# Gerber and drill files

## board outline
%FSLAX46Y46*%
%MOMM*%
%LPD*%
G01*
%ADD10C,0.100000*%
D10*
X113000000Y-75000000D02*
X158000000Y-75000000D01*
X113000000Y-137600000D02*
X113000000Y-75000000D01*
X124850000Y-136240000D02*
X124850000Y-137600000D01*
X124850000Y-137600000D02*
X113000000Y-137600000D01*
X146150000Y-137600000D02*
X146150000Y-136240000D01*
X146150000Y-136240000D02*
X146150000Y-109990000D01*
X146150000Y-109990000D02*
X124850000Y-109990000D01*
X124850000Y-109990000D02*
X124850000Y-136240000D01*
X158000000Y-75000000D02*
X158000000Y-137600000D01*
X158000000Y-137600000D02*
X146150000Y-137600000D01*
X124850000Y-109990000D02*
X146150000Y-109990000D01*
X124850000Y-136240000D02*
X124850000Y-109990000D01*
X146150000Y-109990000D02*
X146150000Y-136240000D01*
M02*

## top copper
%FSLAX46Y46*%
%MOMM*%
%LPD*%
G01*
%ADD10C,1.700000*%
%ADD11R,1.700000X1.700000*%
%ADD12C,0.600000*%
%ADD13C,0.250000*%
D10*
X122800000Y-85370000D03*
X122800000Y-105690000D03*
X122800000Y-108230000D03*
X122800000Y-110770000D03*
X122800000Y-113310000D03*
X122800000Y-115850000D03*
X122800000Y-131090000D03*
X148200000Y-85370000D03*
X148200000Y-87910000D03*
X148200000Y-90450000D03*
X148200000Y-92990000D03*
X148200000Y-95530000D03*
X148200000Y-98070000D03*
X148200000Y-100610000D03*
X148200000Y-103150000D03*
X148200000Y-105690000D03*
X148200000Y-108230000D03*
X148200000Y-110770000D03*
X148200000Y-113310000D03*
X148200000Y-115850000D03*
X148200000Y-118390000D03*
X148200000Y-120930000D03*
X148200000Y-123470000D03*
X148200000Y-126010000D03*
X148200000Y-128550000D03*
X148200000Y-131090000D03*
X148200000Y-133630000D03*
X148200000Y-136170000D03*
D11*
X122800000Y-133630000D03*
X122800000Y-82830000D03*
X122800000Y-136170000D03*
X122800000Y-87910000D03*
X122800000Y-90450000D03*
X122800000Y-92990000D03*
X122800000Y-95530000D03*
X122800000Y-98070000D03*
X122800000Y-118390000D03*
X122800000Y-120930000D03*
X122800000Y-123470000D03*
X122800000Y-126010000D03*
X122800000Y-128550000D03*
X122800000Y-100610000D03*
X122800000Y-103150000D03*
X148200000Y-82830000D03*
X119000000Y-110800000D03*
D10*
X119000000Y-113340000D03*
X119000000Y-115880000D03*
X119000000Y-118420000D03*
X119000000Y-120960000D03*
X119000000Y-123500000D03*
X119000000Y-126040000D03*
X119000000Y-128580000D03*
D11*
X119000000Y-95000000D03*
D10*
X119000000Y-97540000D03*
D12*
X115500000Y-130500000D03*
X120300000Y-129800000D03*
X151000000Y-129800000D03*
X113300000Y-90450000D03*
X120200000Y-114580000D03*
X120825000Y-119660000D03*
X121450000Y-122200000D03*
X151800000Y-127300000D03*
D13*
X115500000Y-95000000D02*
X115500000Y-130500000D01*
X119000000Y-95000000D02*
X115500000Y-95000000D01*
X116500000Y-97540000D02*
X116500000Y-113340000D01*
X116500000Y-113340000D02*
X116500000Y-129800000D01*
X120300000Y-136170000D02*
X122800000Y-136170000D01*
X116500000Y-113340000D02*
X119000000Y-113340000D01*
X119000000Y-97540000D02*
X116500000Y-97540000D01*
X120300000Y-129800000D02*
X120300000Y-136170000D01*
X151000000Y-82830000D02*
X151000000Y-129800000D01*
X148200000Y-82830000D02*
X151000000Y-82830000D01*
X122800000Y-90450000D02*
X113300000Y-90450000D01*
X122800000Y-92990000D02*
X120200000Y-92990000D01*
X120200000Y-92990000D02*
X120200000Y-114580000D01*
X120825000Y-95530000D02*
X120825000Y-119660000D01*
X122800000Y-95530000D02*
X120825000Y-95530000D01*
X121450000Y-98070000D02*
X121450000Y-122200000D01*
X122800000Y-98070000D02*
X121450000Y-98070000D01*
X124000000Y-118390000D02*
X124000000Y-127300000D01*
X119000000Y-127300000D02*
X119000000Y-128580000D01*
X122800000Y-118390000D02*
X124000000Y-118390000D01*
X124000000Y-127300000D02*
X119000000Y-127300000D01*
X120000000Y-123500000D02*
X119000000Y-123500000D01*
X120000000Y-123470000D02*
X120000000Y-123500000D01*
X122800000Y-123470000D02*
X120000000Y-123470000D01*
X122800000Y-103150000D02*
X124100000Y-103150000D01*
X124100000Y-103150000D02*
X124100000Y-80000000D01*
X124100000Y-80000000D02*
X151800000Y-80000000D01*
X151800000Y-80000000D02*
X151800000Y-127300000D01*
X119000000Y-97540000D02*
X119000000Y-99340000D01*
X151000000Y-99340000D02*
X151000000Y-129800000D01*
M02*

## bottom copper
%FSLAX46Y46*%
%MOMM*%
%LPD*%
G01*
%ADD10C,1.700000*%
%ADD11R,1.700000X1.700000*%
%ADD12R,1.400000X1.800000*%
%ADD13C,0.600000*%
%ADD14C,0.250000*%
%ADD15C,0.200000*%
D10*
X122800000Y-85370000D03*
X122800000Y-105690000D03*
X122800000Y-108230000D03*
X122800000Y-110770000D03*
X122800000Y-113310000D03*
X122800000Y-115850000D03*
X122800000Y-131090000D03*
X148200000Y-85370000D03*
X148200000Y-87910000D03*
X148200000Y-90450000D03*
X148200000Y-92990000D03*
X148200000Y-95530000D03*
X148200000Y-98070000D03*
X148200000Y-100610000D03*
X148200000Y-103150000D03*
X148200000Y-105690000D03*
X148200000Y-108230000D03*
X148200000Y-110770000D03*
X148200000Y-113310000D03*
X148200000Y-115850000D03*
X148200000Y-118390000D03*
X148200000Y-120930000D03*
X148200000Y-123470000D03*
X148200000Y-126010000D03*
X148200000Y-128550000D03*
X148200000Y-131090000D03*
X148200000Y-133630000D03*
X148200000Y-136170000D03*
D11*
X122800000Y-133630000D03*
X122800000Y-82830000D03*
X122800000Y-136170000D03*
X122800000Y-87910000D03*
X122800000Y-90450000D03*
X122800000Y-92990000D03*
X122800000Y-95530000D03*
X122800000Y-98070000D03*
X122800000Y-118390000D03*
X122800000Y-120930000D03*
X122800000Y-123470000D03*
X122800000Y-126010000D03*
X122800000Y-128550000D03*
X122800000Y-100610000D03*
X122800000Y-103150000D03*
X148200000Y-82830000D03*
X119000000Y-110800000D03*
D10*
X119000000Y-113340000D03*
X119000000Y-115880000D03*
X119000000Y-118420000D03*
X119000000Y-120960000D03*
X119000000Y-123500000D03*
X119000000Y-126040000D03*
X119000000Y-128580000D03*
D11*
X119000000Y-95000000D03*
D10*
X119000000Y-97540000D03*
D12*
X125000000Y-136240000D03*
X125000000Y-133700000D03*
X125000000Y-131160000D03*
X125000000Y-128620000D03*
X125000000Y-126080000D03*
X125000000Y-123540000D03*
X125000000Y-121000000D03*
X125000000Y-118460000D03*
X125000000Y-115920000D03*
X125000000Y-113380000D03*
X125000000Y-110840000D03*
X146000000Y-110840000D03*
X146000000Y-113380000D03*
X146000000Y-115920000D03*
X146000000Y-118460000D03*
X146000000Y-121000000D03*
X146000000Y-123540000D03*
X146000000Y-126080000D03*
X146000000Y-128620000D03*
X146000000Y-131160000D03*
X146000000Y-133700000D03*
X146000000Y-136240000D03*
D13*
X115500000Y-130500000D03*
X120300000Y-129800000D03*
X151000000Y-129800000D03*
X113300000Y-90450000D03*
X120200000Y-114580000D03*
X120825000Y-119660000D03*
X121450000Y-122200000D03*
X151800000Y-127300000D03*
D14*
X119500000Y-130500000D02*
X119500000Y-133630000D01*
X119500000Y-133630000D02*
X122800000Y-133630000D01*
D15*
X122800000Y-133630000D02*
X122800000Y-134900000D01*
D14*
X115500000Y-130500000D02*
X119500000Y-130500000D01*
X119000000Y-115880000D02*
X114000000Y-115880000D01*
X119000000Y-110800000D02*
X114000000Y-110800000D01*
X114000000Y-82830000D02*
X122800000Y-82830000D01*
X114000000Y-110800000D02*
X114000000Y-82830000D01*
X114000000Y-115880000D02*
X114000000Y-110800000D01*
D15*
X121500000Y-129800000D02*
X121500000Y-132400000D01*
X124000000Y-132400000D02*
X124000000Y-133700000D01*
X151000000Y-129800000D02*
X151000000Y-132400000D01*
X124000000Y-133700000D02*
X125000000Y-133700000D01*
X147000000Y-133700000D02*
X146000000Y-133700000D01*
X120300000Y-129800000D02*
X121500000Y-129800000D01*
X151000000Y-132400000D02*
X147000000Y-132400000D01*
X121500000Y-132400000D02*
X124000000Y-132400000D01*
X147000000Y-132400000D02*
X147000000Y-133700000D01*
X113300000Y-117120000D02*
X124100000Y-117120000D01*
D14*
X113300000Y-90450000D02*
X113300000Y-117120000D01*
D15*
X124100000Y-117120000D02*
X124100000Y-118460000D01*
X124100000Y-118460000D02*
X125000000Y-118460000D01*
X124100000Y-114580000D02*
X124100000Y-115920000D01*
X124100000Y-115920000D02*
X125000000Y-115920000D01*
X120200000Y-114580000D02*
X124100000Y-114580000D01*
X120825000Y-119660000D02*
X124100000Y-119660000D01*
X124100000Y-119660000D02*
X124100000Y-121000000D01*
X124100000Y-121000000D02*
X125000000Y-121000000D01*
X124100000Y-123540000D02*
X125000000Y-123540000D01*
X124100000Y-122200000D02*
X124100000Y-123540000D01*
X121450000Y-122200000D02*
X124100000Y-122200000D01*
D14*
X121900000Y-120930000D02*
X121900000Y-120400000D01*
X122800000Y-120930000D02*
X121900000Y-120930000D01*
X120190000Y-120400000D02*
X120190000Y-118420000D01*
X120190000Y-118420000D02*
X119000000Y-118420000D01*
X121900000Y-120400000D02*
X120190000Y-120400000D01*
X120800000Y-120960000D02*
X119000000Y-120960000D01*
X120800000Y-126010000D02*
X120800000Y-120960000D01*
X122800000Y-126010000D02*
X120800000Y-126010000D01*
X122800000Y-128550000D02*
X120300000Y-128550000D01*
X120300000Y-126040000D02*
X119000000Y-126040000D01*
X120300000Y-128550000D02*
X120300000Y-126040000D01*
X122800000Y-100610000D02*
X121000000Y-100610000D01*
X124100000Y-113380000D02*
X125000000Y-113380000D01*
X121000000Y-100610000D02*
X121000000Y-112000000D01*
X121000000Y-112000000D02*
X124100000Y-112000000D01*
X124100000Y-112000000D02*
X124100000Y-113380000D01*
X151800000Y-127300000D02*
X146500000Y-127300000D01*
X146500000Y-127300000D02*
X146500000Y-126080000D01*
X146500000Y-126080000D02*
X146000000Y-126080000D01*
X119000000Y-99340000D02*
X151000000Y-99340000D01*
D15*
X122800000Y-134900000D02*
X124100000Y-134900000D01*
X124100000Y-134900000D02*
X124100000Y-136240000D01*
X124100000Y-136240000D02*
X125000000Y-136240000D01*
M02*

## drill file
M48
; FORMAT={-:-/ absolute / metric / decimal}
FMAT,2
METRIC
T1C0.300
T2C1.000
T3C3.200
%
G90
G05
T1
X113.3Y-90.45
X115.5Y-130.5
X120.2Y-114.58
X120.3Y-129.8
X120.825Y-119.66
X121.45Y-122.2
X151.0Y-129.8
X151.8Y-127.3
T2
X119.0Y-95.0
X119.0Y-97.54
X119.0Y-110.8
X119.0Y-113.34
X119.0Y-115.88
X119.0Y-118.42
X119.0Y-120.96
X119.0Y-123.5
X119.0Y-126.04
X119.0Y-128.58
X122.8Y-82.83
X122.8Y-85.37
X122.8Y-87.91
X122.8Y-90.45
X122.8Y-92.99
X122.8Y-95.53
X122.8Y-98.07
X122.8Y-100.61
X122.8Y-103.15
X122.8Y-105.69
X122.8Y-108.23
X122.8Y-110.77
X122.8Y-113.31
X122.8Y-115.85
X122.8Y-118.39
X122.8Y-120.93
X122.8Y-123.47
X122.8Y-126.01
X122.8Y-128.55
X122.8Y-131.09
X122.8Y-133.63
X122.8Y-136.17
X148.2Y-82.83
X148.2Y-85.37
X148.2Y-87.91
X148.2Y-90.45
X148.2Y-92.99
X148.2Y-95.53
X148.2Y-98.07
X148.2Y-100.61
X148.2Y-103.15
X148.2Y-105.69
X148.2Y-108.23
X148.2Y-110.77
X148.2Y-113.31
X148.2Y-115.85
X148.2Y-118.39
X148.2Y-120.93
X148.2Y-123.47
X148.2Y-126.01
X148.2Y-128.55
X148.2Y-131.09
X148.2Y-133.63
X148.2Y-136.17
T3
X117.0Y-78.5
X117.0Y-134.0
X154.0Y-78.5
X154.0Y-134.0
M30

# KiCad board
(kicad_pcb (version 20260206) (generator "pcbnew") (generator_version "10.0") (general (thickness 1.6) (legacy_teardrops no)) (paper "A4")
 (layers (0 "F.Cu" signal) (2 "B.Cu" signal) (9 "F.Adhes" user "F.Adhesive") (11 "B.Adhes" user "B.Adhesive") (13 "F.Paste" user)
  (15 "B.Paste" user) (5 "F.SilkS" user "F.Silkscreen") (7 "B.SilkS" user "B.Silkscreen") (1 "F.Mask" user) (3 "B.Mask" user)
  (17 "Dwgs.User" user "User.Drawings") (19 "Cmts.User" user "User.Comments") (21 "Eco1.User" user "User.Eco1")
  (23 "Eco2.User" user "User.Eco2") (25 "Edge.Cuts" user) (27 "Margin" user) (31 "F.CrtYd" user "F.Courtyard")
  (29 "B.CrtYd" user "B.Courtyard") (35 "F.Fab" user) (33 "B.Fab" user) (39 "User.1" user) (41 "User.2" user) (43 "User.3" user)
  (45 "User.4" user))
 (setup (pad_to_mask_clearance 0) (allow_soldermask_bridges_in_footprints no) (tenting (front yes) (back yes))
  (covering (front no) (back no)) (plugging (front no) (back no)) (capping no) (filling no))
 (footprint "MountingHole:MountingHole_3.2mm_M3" (layer "F.Cu") (at 117 78.5)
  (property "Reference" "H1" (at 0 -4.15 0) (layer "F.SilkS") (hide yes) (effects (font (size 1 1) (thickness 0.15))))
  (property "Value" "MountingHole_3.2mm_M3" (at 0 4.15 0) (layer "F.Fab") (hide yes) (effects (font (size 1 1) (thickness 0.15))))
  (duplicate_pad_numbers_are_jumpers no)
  (pad "" np_thru_hole circle (at 0 0) (size 3.2 3.2) (drill 3.2) (layers "*.Cu" "*.Mask")))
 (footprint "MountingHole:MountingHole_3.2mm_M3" (layer "F.Cu") (at 117 134)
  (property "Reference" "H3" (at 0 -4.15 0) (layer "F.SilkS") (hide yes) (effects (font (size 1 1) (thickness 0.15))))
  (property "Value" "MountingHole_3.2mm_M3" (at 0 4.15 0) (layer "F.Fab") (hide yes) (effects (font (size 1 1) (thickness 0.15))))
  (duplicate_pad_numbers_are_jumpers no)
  (pad "" np_thru_hole circle (at 0 0) (size 3.2 3.2) (drill 3.2) (layers "*.Cu" "*.Mask")))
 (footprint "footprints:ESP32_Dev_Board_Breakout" (layer "F.Cu") (at 121.53 81.98)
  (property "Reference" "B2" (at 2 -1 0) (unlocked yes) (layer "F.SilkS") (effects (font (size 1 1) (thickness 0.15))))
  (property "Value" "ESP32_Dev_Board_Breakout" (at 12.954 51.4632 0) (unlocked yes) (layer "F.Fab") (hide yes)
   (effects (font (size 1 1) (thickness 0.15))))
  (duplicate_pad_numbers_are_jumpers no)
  (pad "" thru_hole circle (at 1.27 3.39 90) (size 1.7 1.7) (drill 1) (layers "*.Cu" "*.Mask") (remove_unused_layers no))
  (pad "" thru_hole circle (at 1.27 23.71 90) (size 1.7 1.7) (drill 1) (layers "*.Cu" "*.Mask") (remove_unused_layers no))
  (pad "" thru_hole circle (at 1.27 26.25 90) (size 1.7 1.7) (drill 1) (layers "*.Cu" "*.Mask") (remove_unused_layers no))
  (pad "" thru_hole circle (at 1.27 28.79 90) (size 1.7 1.7) (drill 1) (layers "*.Cu" "*.Mask") (remove_unused_layers no))
  (pad "" thru_hole circle (at 1.27 31.33 90) (size 1.7 1.7) (drill 1) (layers "*.Cu" "*.Mask") (remove_unused_layers no))
  (pad "" thru_hole circle (at 1.27 33.87 90) (size 1.7 1.7) (drill 1) (layers "*.Cu" "*.Mask") (remove_unused_layers no))
  (pad "" thru_hole circle (at 1.27 49.11 90) (size 1.7 1.7) (drill 1) (layers "*.Cu" "*.Mask") (remove_unused_layers no))
  (pad "" thru_hole circle (at 26.67 3.39 270) (size 1.7 1.7) (drill 1) (layers "*.Cu" "*.Mask") (remove_unused_layers no))
  (pad "" thru_hole circle (at 26.67 5.93 270) (size 1.7 1.7) (drill 1) (layers "*.Cu" "*.Mask") (remove_unused_layers no))
  (pad "" thru_hole circle (at 26.67 8.47 270) (size 1.7 1.7) (drill 1) (layers "*.Cu" "*.Mask") (remove_unused_layers no))
  (pad "" thru_hole circle (at 26.67 11.01 270) (size 1.7 1.7) (drill 1) (layers "*.Cu" "*.Mask") (remove_unused_layers no))
  (pad "" thru_hole circle (at 26.67 13.55 270) (size 1.7 1.7) (drill 1) (layers "*.Cu" "*.Mask") (remove_unused_layers no))
  (pad "" thru_hole circle (at 26.67 16.09 270) (size 1.7 1.7) (drill 1) (layers "*.Cu" "*.Mask") (remove_unused_layers no))
  (pad "" thru_hole circle (at 26.67 18.63 270) (size 1.7 1.7) (drill 1) (layers "*.Cu" "*.Mask") (remove_unused_layers no))
  (pad "" thru_hole circle (at 26.67 21.17 270) (size 1.7 1.7) (drill 1) (layers "*.Cu" "*.Mask") (remove_unused_layers no))
  (pad "" thru_hole circle (at 26.67 23.71 270) (size 1.7 1.7) (drill 1) (layers "*.Cu" "*.Mask") (remove_unused_layers no))
  (pad "" thru_hole circle (at 26.67 26.25 270) (size 1.7 1.7) (drill 1) (layers "*.Cu" "*.Mask") (remove_unused_layers no))
  (pad "" thru_hole circle (at 26.67 28.79 270) (size 1.7 1.7) (drill 1) (layers "*.Cu" "*.Mask") (remove_unused_layers no))
  (pad "" thru_hole circle (at 26.67 31.33 270) (size 1.7 1.7) (drill 1) (layers "*.Cu" "*.Mask") (remove_unused_layers no))
  (pad "" thru_hole circle (at 26.67 33.87 270) (size 1.7 1.7) (drill 1) (layers "*.Cu" "*.Mask") (remove_unused_layers no))
  (pad "" thru_hole circle (at 26.67 36.41 270) (size 1.7 1.7) (drill 1) (layers "*.Cu" "*.Mask") (remove_unused_layers no))
  (pad "" thru_hole circle (at 26.67 38.95 270) (size 1.7 1.7) (drill 1) (layers "*.Cu" "*.Mask") (remove_unused_layers no))
  (pad "" thru_hole circle (at 26.67 41.49 270) (size 1.7 1.7) (drill 1) (layers "*.Cu" "*.Mask") (remove_unused_layers no))
  (pad "" thru_hole circle (at 26.67 44.03 270) (size 1.7 1.7) (drill 1) (layers "*.Cu" "*.Mask") (remove_unused_layers no))
  (pad "" thru_hole circle (at 26.67 46.57 270) (size 1.7 1.7) (drill 1) (layers "*.Cu" "*.Mask") (remove_unused_layers no))
  (pad "" thru_hole circle (at 26.67 49.11 270) (size 1.7 1.7) (drill 1) (layers "*.Cu" "*.Mask") (remove_unused_layers no))
  (pad "" thru_hole circle (at 26.67 51.65 270) (size 1.7 1.7) (drill 1) (layers "*.Cu" "*.Mask") (remove_unused_layers no))
  (pad "" thru_hole circle (at 26.67 54.19 270) (size 1.7 1.7) (drill 1) (layers "*.Cu" "*.Mask") (remove_unused_layers no))
  (pad "1" thru_hole rect (at 1.27 51.65 90) (size 1.7 1.7) (drill 1) (layers "*.Cu" "*.Mask") (remove_unused_layers no) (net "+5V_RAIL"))
  (pad "2" thru_hole rect (at 1.27 0.85 90) (size 1.7 1.7) (drill 1) (layers "*.Cu" "*.Mask") (remove_unused_layers no) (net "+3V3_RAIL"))
  (pad "3" thru_hole rect (at 1.27 54.19 90) (size 1.7 1.7) (drill 1) (layers "*.Cu" "*.Mask") (remove_unused_layers no) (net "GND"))
  (pad "4" thru_hole rect (at 1.27 5.93 90) (size 1.7 1.7) (drill 1) (layers "*.Cu" "*.Mask") (remove_unused_layers no)
   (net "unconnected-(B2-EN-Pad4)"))
  (pad "5" thru_hole rect (at 1.27 8.47 90) (size 1.7 1.7) (drill 1) (layers "*.Cu" "*.Mask") (remove_unused_layers no)
   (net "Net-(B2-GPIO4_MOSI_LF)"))
  (pad "6" thru_hole rect (at 1.27 11.01 90) (size 1.7 1.7) (drill 1) (layers "*.Cu" "*.Mask") (remove_unused_layers no)
   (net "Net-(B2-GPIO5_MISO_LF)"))
  (pad "7" thru_hole rect (at 1.27 13.55 90) (size 1.7 1.7) (drill 1) (layers "*.Cu" "*.Mask") (remove_unused_layers no)
   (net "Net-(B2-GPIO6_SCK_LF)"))
  (pad "8" thru_hole rect (at 1.27 16.09 90) (size 1.7 1.7) (drill 1) (layers "*.Cu" "*.Mask") (remove_unused_layers no)
   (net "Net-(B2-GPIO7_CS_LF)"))
  (pad "9" thru_hole rect (at 1.27 36.41 90) (size 1.7 1.7) (drill 1) (layers "*.Cu" "*.Mask") (remove_unused_layers no)
   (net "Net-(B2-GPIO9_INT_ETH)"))
  (pad "10" thru_hole rect (at 1.27 38.95 90) (size 1.7 1.7) (drill 1) (layers "*.Cu" "*.Mask") (remove_unused_layers no)
   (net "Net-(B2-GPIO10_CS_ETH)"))
  (pad "11" thru_hole rect (at 1.27 41.49 90) (size 1.7 1.7) (drill 1) (layers "*.Cu" "*.Mask") (remove_unused_layers no)
   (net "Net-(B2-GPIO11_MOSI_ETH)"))
  (pad "12" thru_hole rect (at 1.27 44.03 90) (size 1.7 1.7) (drill 1) (layers "*.Cu" "*.Mask") (remove_unused_layers no)
   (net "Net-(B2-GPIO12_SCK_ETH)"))
  (pad "13" thru_hole rect (at 1.27 46.57 90) (size 1.7 1.7) (drill 1) (layers "*.Cu" "*.Mask") (remove_unused_layers no)
   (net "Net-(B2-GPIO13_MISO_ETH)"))
  (pad "14" thru_hole rect (at 1.27 18.63 90) (size 1.7 1.7) (drill 1) (layers "*.Cu" "*.Mask") (remove_unused_layers no)
   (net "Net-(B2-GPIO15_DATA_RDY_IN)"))
  (pad "15" thru_hole rect (at 1.27 21.17 90) (size 1.7 1.7) (drill 1) (layers "*.Cu" "*.Mask") (remove_unused_layers no)
   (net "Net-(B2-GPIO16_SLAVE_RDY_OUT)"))
  (pad "16" thru_hole rect (at 26.67 0.85 270) (size 1.7 1.7) (drill 1) (layers "*.Cu" "*.Mask") (remove_unused_layers no) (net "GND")))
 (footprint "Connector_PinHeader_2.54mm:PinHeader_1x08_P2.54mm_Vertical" (layer "F.Cu") (at 119 110.8)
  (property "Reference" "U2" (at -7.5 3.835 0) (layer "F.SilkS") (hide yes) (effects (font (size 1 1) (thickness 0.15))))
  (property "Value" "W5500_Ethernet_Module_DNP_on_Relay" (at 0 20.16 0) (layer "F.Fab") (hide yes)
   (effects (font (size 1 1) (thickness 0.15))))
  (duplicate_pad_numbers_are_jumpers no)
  (pad "1" thru_hole rect (at 0 0) (size 1.7 1.7) (drill 1) (layers "*.Cu" "*.Mask") (remove_unused_layers no) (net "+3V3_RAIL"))
  (pad "2" thru_hole circle (at 0 2.54) (size 1.7 1.7) (drill 1) (layers "*.Cu" "*.Mask") (remove_unused_layers no) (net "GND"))
  (pad "3" thru_hole circle (at 0 5.08) (size 1.7 1.7) (drill 1) (layers "*.Cu" "*.Mask") (remove_unused_layers no) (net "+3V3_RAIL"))
  (pad "4" thru_hole circle (at 0 7.62) (size 1.7 1.7) (drill 1) (layers "*.Cu" "*.Mask") (remove_unused_layers no)
   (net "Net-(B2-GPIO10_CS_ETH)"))
  (pad "5" thru_hole circle (at 0 10.16) (size 1.7 1.7) (drill 1) (layers "*.Cu" "*.Mask") (remove_unused_layers no)
   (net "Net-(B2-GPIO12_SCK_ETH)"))
  (pad "6" thru_hole circle (at 0 12.7) (size 1.7 1.7) (drill 1) (layers "*.Cu" "*.Mask") (remove_unused_layers no)
   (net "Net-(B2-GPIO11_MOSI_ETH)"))
  (pad "7" thru_hole circle (at 0 15.24) (size 1.7 1.7) (drill 1) (layers "*.Cu" "*.Mask") (remove_unused_layers no)
   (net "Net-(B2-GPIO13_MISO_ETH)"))
  (pad "8" thru_hole circle (at 0 17.78) (size 1.7 1.7) (drill 1) (layers "*.Cu" "*.Mask") (remove_unused_layers no)
   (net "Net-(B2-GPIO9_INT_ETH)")))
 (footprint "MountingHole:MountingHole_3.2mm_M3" (layer "F.Cu") (at 154 134)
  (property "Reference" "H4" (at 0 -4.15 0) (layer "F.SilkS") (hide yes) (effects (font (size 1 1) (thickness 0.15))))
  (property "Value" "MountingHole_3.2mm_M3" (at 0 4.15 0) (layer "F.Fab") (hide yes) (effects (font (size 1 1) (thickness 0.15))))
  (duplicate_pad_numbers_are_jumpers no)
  (pad "" np_thru_hole circle (at 0 0) (size 3.2 3.2) (drill 3.2) (layers "*.Cu" "*.Mask")))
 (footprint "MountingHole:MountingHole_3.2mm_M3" (layer "F.Cu") (at 154 78.5)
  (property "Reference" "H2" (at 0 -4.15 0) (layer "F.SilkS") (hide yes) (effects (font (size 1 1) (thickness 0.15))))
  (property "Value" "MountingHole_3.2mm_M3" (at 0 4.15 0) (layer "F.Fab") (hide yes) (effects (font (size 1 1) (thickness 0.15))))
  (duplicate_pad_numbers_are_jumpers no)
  (pad "" np_thru_hole circle (at 0 0) (size 3.2 3.2) (drill 3.2) (layers "*.Cu" "*.Mask")))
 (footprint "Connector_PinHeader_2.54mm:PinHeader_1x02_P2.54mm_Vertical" (layer "F.Cu") (at 119 95)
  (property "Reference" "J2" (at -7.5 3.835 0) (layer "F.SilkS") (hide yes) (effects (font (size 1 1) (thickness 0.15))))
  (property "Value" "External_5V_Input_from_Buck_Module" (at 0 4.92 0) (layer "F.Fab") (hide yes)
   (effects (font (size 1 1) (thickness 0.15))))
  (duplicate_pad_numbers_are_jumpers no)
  (pad "1" thru_hole rect (at 0 0) (size 1.7 1.7) (drill 1) (layers "*.Cu" "*.Mask") (remove_unused_layers no) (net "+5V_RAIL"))
  (pad "2" thru_hole circle (at 0 2.54) (size 1.7 1.7) (drill 1) (layers "*.Cu" "*.Mask") (remove_unused_layers no) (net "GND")))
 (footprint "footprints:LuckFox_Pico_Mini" (layer "B.Cu") (at 125 110.14)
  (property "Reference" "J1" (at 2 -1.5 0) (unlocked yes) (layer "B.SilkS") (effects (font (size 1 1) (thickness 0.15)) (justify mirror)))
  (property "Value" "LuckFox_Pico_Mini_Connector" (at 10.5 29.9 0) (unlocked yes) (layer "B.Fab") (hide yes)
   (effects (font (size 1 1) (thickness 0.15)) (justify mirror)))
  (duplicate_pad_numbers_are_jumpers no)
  (fp_line (start -0.15 -0.15) (end 21.15 -0.15) (stroke (width 0.1) (type solid)) (layer "Edge.Cuts"))
  (fp_line (start -0.15 26.1) (end -0.15 -0.15) (stroke (width 0.1) (type solid)) (layer "Edge.Cuts"))
  (fp_line (start 21.15 -0.15) (end 21.15 26.1) (stroke (width 0.1) (type solid)) (layer "Edge.Cuts"))
  (pad "1" smd rect (at 0 26.1 90) (size 1.8 1.4) (layers "B.Cu" "B.Mask" "B.Paste") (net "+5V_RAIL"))
  (pad "2" smd rect (at 0 23.56 90) (size 1.8 1.4) (layers "B.Cu" "B.Mask" "B.Paste") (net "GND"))
  (pad "3" smd rect (at 0 21.02 90) (size 1.8 1.4) (layers "B.Cu" "B.Mask" "B.Paste") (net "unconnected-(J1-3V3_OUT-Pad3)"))
  (pad "4" smd rect (at 0 18.48 90) (size 1.8 1.4) (layers "B.Cu" "B.Mask" "B.Paste") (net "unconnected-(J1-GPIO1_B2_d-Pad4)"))
  (pad "5" smd rect (at 0 15.94 90) (size 1.8 1.4) (layers "B.Cu" "B.Mask" "B.Paste") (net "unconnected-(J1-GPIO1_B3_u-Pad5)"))
  (pad "6" smd rect (at 0 13.4 90) (size 1.8 1.4) (layers "B.Cu" "B.Mask" "B.Paste") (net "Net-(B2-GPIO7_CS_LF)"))
  (pad "7" smd rect (at 0 10.86 90) (size 1.8 1.4) (layers "B.Cu" "B.Mask" "B.Paste") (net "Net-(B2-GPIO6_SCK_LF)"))
  (pad "8" smd rect (at 0 8.32 90) (size 1.8 1.4) (layers "B.Cu" "B.Mask" "B.Paste") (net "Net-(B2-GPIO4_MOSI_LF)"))
  (pad "9" smd rect (at 0 5.78 90) (size 1.8 1.4) (layers "B.Cu" "B.Mask" "B.Paste") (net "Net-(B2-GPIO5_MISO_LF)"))
  (pad "10" smd rect (at 0 3.24 90) (size 1.8 1.4) (layers "B.Cu" "B.Mask" "B.Paste") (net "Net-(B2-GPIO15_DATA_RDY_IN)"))
  (pad "11" smd rect (at 0 0.7 90) (size 1.8 1.4) (layers "B.Cu" "B.Mask" "B.Paste") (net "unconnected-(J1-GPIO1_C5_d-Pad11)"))
  (pad "12" smd rect (at 21 0.7 90) (size 1.8 1.4) (layers "B.Cu" "B.Mask" "B.Paste") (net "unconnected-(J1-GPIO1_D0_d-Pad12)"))
  (pad "13" smd rect (at 21 3.24 90) (size 1.8 1.4) (layers "B.Cu" "B.Mask" "B.Paste") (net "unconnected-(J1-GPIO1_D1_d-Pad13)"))
  (pad "14" smd rect (at 21 5.78 90) (size 1.8 1.4) (layers "B.Cu" "B.Mask" "B.Paste") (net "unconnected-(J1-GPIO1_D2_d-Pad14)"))
  (pad "15" smd rect (at 21 8.32 90) (size 1.8 1.4) (layers "B.Cu" "B.Mask" "B.Paste") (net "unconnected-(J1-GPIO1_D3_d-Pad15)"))
  (pad "16" smd rect (at 21 10.86 90) (size 1.8 1.4) (layers "B.Cu" "B.Mask" "B.Paste") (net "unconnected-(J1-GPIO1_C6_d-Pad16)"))
  (pad "17" smd rect (at 21 13.4 90) (size 1.8 1.4) (layers "B.Cu" "B.Mask" "B.Paste") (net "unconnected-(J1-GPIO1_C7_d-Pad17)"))
  (pad "18" smd rect (at 21 15.94 90) (size 1.8 1.4) (layers "B.Cu" "B.Mask" "B.Paste") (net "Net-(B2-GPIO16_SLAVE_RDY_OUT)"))
  (pad "19" smd rect (at 21 18.48 90) (size 1.8 1.4) (layers "B.Cu" "B.Mask" "B.Paste") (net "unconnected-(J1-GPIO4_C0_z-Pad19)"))
  (pad "20" smd rect (at 21 21.02 90) (size 1.8 1.4) (layers "B.Cu" "B.Mask" "B.Paste") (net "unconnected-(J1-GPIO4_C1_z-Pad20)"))
  (pad "21" smd rect (at 21 23.56 90) (size 1.8 1.4) (layers "B.Cu" "B.Mask" "B.Paste") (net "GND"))
  (pad "22" smd rect (at 21 26.1 90) (size 1.8 1.4) (layers "B.Cu" "B.Mask" "B.Paste") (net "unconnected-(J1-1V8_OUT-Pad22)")))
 (gr_line (start 113 75) (end 158 75) (stroke (width 0.1) (type solid)) (layer "Edge.Cuts"))
 (gr_line (start 113 137.6) (end 113 75) (stroke (width 0.1) (type solid)) (layer "Edge.Cuts"))
 (gr_line (start 124.85 136.24) (end 124.85 137.6) (stroke (width 0.1) (type solid)) (layer "Edge.Cuts"))
 (gr_line (start 124.85 137.6) (end 113 137.6) (stroke (width 0.1) (type solid)) (layer "Edge.Cuts"))
 (gr_line (start 146.15 137.6) (end 146.15 136.24) (stroke (width 0.1) (type solid)) (layer "Edge.Cuts"))
 (gr_line (start 146.15 136.24) (end 146.15 109.99) (stroke (width 0.1) (type solid)) (layer "Edge.Cuts"))
 (gr_line (start 146.15 109.99) (end 124.85 109.99) (stroke (width 0.1) (type solid)) (layer "Edge.Cuts"))
 (gr_line (start 124.85 109.99) (end 124.85 136.24) (stroke (width 0.1) (type solid)) (layer "Edge.Cuts"))
 (gr_line (start 158 75) (end 158 137.6) (stroke (width 0.1) (type solid)) (layer "Edge.Cuts"))
 (gr_line (start 158 137.6) (end 146.15 137.6) (stroke (width 0.1) (type solid)) (layer "Edge.Cuts"))
 (segment (start 115.5 95) (end 115.5 130.5) (width 0.25) (layer "F.Cu") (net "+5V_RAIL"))
 (segment (start 119 95) (end 115.5 95) (width 0.25) (layer "F.Cu") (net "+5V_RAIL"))
 (via (at 115.5 130.5) (size 0.6) (drill 0.3) (layers "F.Cu" "B.Cu") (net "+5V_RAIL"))
 (segment (start 119.5 130.5) (end 119.5 133.63) (width 0.25) (layer "B.Cu") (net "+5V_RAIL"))
 (segment (start 119.5 133.63) (end 122.8 133.63) (width 0.25) (layer "B.Cu") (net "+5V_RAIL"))
 (segment (start 122.8 133.63) (end 122.8 134.9) (width 0.2) (layer "B.Cu") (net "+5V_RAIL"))
 (segment (start 115.5 130.5) (end 119.5 130.5) (width 0.25) (layer "B.Cu") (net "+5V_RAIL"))
 (segment (start 119 115.88) (end 114 115.88) (width 0.25) (layer "B.Cu") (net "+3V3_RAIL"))
 (segment (start 119 110.8) (end 114 110.8) (width 0.25) (layer "B.Cu") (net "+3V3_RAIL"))
 (segment (start 114 82.83) (end 122.8 82.83) (width 0.25) (layer "B.Cu") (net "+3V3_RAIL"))
 (segment (start 114 110.8) (end 114 82.83) (width 0.25) (layer "B.Cu") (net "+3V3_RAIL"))
 (segment (start 114 115.88) (end 114 110.8) (width 0.25) (layer "B.Cu") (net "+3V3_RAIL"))
 (segment (start 116.5 97.54) (end 116.5 113.34) (width 0.25) (layer "F.Cu") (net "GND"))
 (segment (start 116.5 113.34) (end 116.5 129.8) (width 0.25) (layer "F.Cu") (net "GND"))
 (segment (start 120.3 136.17) (end 122.8 136.17) (width 0.25) (layer "F.Cu") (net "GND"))
 (segment (start 116.5 113.34) (end 119 113.34) (width 0.25) (layer "F.Cu") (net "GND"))
 (segment (start 119 97.54) (end 116.5 97.54) (width 0.25) (layer "F.Cu") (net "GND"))
 (segment (start 120.3 129.8) (end 120.3 136.17) (width 0.25) (layer "F.Cu") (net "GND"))
 (segment (start 151 82.83) (end 151 129.8) (width 0.25) (layer "F.Cu") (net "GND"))
 (segment (start 148.2 82.83) (end 151 82.83) (width 0.25) (layer "F.Cu") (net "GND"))
 (via (at 120.3 129.8) (size 0.6) (drill 0.3) (layers "F.Cu" "B.Cu") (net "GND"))
 (via (at 151 129.8) (size 0.6) (drill 0.3) (layers "F.Cu" "B.Cu") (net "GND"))
 (segment (start 121.5 129.8) (end 121.5 132.4) (width 0.2) (layer "B.Cu") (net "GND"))
 (segment (start 124 132.4) (end 124 133.7) (width 0.2) (layer "B.Cu") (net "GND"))
 (segment (start 151 129.8) (end 151 132.4) (width 0.2) (layer "B.Cu") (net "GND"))
 (segment (start 124 133.7) (end 125 133.7) (width 0.2) (layer "B.Cu") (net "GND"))
 (segment (start 147 133.7) (end 146 133.7) (width 0.2) (layer "B.Cu") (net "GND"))
 (segment (start 120.3 129.8) (end 121.5 129.8) (width 0.2) (layer "B.Cu") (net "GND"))
 (segment (start 151 132.4) (end 147 132.4) (width 0.2) (layer "B.Cu") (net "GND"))
 (segment (start 121.5 132.4) (end 124 132.4) (width 0.2) (layer "B.Cu") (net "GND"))
 (segment (start 147 132.4) (end 147 133.7) (width 0.2) (layer "B.Cu") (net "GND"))
 (segment (start 122.8 90.45) (end 113.3 90.45) (width 0.25) (layer "F.Cu") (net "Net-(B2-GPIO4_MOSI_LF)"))
 (via (at 113.3 90.45) (size 0.6) (drill 0.3) (layers "F.Cu" "B.Cu") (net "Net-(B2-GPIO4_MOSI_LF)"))
 (segment (start 113.3 117.12) (end 124.1 117.12) (width 0.2) (layer "B.Cu") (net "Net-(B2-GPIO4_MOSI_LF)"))
 (segment (start 113.3 90.45) (end 113.3 117.12) (width 0.25) (layer "B.Cu") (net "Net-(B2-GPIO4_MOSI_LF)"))
 (segment (start 124.1 117.12) (end 124.1 118.46) (width 0.2) (layer "B.Cu") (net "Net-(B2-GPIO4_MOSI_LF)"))
 (segment (start 124.1 118.46) (end 125 118.46) (width 0.2) (layer "B.Cu") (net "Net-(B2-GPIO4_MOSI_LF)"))
 (segment (start 122.8 92.99) (end 120.2 92.99) (width 0.25) (layer "F.Cu") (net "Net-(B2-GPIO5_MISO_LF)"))
 (segment (start 120.2 92.99) (end 120.2 114.58) (width 0.25) (layer "F.Cu") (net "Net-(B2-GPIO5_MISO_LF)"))
 (via (at 120.2 114.58) (size 0.6) (drill 0.3) (layers "F.Cu" "B.Cu") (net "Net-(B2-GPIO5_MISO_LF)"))
 (segment (start 124.1 114.58) (end 124.1 115.92) (width 0.2) (layer "B.Cu") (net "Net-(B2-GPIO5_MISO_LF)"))
 (segment (start 124.1 115.92) (end 125 115.92) (width 0.2) (layer "B.Cu") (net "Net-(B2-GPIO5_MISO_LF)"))
 (segment (start 120.2 114.58) (end 124.1 114.58) (width 0.2) (layer "B.Cu") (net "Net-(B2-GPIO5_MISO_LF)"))
 (segment (start 120.825 95.53) (end 120.825 119.66) (width 0.25) (layer "F.Cu") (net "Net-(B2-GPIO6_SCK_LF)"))
 (segment (start 122.8 95.53) (end 120.825 95.53) (width 0.25) (layer "F.Cu") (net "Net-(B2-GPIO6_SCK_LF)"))
 (via (at 120.825 119.66) (size 0.6) (drill 0.3) (layers "F.Cu" "B.Cu") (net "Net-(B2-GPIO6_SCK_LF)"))
 (segment (start 120.825 119.66) (end 124.1 119.66) (width 0.2) (layer "B.Cu") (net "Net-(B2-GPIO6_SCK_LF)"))
 (segment (start 124.1 119.66) (end 124.1 121) (width 0.2) (layer "B.Cu") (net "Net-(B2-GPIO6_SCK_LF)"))
 (segment (start 124.1 121) (end 125 121) (width 0.2) (layer "B.Cu") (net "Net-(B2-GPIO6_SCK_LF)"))
 (segment (start 121.45 98.07) (end 121.45 122.2) (width 0.25) (layer "F.Cu") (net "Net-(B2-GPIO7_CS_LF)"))
 (segment (start 122.8 98.07) (end 121.45 98.07) (width 0.25) (layer "F.Cu") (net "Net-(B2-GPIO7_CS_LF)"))
 (via (at 121.45 122.2) (size 0.6) (drill 0.3) (layers "F.Cu" "B.Cu") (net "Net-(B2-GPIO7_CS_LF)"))
 (segment (start 124.1 123.54) (end 125 123.54) (width 0.2) (layer "B.Cu") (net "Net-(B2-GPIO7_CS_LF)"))
 (segment (start 124.1 122.2) (end 124.1 123.54) (width 0.2) (layer "B.Cu") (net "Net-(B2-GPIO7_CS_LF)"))
 (segment (start 121.45 122.2) (end 124.1 122.2) (width 0.2) (layer "B.Cu") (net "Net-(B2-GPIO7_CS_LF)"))
 (segment (start 124 118.39) (end 124 127.3) (width 0.25) (layer "F.Cu") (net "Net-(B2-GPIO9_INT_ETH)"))
 (segment (start 119 127.3) (end 119 128.58) (width 0.25) (layer "F.Cu") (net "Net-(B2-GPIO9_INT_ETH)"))
 (segment (start 122.8 118.39) (end 124 118.39) (width 0.25) (layer "F.Cu") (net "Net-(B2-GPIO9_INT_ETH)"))
 (segment (start 124 127.3) (end 119 127.3) (width 0.25) (layer "F.Cu") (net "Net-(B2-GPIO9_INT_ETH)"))
 (segment (start 121.9 120.93) (end 121.9 120.4) (width 0.25) (layer "B.Cu") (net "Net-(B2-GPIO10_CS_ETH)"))
 (segment (start 122.8 120.93) (end 121.9 120.93) (width 0.25) (layer "B.Cu") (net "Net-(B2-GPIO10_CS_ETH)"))
 (segment (start 120.19 120.4) (end 120.19 118.42) (width 0.25) (layer "B.Cu") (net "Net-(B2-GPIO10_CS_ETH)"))
 (segment (start 120.19 118.42) (end 119 118.42) (width 0.25) (layer "B.Cu") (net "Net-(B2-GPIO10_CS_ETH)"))
 (segment (start 121.9 120.4) (end 120.19 120.4) (width 0.25) (layer "B.Cu") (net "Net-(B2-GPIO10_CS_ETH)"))
 (segment (start 120 123.5) (end 119 123.5) (width 0.25) (layer "F.Cu") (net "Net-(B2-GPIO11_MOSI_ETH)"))
 (segment (start 120 123.47) (end 120 123.5) (width 0.25) (layer "F.Cu") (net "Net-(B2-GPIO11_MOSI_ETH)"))
 (segment (start 122.8 123.47) (end 120 123.47) (width 0.25) (layer "F.Cu") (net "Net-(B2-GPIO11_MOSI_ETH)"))
 (segment (start 120.8 120.96) (end 119 120.96) (width 0.25) (layer "B.Cu") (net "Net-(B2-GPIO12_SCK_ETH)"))
 (segment (start 120.8 126.01) (end 120.8 120.96) (width 0.25) (layer "B.Cu") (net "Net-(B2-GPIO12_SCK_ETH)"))
 (segment (start 122.8 126.01) (end 120.8 126.01) (width 0.25) (layer "B.Cu") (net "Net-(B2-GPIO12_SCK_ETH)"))
 (segment (start 122.8 128.55) (end 120.3 128.55) (width 0.25) (layer "B.Cu") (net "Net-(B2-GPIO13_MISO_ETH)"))
 (segment (start 120.3 126.04) (end 119 126.04) (width 0.25) (layer "B.Cu") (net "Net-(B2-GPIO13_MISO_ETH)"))
 (segment (start 120.3 128.55) (end 120.3 126.04) (width 0.25) (layer "B.Cu") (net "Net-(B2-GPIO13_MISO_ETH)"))
 (segment (start 122.8 100.61) (end 121 100.61) (width 0.25) (layer "B.Cu") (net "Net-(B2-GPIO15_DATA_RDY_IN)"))
 (segment (start 124.1 113.38) (end 125 113.38) (width 0.25) (layer "B.Cu") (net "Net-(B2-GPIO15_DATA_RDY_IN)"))
 (segment (start 121 100.61) (end 121 112) (width 0.25) (layer "B.Cu") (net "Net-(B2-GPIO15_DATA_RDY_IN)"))
 (segment (start 121 112) (end 124.1 112) (width 0.25) (layer "B.Cu") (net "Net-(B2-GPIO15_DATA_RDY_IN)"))
 (segment (start 124.1 112) (end 124.1 113.38) (width 0.25) (layer "B.Cu") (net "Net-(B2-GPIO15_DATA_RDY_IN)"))
 (segment (start 122.8 103.15) (end 124.1 103.15) (width 0.25) (layer "F.Cu") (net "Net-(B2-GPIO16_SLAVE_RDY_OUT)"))
 (segment (start 124.1 103.15) (end 124.1 80) (width 0.25) (layer "F.Cu") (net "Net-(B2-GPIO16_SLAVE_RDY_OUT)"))
 (segment (start 124.1 80) (end 151.8 80) (width 0.25) (layer "F.Cu") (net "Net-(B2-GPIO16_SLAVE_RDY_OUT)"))
 (segment (start 151.8 80) (end 151.8 127.3) (width 0.25) (layer "F.Cu") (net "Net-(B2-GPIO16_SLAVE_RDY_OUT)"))
 (via (at 151.8 127.3) (size 0.6) (drill 0.3) (layers "F.Cu" "B.Cu") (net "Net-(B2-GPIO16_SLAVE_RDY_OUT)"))
 (segment (start 151.8 127.3) (end 146.5 127.3) (width 0.25) (layer "B.Cu") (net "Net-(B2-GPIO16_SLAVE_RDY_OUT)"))
 (segment (start 146.5 127.3) (end 146.5 126.08) (width 0.25) (layer "B.Cu") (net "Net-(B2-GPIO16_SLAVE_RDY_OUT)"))
 (segment (start 146.5 126.08) (end 146 126.08) (width 0.25) (layer "B.Cu") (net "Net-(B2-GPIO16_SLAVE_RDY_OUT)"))
 (segment (start 119.0 97.54) (end 119.0 99.34) (width 0.25) (layer "F.Cu") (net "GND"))
 (segment (start 119.0 99.34) (end 151.0 99.34) (width 0.25) (layer "B.Cu") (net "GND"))
 (segment (start 151.0 99.34) (end 151.0 129.8) (width 0.25) (layer "F.Cu") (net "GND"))
 (segment (start 122.8 134.9) (end 124.1 134.9) (width 0.2) (layer "B.Cu") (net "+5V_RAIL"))
 (segment (start 124.1 134.9) (end 124.1 136.24) (width 0.2) (layer "B.Cu") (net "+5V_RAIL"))
 (segment (start 124.1 136.24) (end 125.0 136.24) (width 0.2) (layer "B.Cu") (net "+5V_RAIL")))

